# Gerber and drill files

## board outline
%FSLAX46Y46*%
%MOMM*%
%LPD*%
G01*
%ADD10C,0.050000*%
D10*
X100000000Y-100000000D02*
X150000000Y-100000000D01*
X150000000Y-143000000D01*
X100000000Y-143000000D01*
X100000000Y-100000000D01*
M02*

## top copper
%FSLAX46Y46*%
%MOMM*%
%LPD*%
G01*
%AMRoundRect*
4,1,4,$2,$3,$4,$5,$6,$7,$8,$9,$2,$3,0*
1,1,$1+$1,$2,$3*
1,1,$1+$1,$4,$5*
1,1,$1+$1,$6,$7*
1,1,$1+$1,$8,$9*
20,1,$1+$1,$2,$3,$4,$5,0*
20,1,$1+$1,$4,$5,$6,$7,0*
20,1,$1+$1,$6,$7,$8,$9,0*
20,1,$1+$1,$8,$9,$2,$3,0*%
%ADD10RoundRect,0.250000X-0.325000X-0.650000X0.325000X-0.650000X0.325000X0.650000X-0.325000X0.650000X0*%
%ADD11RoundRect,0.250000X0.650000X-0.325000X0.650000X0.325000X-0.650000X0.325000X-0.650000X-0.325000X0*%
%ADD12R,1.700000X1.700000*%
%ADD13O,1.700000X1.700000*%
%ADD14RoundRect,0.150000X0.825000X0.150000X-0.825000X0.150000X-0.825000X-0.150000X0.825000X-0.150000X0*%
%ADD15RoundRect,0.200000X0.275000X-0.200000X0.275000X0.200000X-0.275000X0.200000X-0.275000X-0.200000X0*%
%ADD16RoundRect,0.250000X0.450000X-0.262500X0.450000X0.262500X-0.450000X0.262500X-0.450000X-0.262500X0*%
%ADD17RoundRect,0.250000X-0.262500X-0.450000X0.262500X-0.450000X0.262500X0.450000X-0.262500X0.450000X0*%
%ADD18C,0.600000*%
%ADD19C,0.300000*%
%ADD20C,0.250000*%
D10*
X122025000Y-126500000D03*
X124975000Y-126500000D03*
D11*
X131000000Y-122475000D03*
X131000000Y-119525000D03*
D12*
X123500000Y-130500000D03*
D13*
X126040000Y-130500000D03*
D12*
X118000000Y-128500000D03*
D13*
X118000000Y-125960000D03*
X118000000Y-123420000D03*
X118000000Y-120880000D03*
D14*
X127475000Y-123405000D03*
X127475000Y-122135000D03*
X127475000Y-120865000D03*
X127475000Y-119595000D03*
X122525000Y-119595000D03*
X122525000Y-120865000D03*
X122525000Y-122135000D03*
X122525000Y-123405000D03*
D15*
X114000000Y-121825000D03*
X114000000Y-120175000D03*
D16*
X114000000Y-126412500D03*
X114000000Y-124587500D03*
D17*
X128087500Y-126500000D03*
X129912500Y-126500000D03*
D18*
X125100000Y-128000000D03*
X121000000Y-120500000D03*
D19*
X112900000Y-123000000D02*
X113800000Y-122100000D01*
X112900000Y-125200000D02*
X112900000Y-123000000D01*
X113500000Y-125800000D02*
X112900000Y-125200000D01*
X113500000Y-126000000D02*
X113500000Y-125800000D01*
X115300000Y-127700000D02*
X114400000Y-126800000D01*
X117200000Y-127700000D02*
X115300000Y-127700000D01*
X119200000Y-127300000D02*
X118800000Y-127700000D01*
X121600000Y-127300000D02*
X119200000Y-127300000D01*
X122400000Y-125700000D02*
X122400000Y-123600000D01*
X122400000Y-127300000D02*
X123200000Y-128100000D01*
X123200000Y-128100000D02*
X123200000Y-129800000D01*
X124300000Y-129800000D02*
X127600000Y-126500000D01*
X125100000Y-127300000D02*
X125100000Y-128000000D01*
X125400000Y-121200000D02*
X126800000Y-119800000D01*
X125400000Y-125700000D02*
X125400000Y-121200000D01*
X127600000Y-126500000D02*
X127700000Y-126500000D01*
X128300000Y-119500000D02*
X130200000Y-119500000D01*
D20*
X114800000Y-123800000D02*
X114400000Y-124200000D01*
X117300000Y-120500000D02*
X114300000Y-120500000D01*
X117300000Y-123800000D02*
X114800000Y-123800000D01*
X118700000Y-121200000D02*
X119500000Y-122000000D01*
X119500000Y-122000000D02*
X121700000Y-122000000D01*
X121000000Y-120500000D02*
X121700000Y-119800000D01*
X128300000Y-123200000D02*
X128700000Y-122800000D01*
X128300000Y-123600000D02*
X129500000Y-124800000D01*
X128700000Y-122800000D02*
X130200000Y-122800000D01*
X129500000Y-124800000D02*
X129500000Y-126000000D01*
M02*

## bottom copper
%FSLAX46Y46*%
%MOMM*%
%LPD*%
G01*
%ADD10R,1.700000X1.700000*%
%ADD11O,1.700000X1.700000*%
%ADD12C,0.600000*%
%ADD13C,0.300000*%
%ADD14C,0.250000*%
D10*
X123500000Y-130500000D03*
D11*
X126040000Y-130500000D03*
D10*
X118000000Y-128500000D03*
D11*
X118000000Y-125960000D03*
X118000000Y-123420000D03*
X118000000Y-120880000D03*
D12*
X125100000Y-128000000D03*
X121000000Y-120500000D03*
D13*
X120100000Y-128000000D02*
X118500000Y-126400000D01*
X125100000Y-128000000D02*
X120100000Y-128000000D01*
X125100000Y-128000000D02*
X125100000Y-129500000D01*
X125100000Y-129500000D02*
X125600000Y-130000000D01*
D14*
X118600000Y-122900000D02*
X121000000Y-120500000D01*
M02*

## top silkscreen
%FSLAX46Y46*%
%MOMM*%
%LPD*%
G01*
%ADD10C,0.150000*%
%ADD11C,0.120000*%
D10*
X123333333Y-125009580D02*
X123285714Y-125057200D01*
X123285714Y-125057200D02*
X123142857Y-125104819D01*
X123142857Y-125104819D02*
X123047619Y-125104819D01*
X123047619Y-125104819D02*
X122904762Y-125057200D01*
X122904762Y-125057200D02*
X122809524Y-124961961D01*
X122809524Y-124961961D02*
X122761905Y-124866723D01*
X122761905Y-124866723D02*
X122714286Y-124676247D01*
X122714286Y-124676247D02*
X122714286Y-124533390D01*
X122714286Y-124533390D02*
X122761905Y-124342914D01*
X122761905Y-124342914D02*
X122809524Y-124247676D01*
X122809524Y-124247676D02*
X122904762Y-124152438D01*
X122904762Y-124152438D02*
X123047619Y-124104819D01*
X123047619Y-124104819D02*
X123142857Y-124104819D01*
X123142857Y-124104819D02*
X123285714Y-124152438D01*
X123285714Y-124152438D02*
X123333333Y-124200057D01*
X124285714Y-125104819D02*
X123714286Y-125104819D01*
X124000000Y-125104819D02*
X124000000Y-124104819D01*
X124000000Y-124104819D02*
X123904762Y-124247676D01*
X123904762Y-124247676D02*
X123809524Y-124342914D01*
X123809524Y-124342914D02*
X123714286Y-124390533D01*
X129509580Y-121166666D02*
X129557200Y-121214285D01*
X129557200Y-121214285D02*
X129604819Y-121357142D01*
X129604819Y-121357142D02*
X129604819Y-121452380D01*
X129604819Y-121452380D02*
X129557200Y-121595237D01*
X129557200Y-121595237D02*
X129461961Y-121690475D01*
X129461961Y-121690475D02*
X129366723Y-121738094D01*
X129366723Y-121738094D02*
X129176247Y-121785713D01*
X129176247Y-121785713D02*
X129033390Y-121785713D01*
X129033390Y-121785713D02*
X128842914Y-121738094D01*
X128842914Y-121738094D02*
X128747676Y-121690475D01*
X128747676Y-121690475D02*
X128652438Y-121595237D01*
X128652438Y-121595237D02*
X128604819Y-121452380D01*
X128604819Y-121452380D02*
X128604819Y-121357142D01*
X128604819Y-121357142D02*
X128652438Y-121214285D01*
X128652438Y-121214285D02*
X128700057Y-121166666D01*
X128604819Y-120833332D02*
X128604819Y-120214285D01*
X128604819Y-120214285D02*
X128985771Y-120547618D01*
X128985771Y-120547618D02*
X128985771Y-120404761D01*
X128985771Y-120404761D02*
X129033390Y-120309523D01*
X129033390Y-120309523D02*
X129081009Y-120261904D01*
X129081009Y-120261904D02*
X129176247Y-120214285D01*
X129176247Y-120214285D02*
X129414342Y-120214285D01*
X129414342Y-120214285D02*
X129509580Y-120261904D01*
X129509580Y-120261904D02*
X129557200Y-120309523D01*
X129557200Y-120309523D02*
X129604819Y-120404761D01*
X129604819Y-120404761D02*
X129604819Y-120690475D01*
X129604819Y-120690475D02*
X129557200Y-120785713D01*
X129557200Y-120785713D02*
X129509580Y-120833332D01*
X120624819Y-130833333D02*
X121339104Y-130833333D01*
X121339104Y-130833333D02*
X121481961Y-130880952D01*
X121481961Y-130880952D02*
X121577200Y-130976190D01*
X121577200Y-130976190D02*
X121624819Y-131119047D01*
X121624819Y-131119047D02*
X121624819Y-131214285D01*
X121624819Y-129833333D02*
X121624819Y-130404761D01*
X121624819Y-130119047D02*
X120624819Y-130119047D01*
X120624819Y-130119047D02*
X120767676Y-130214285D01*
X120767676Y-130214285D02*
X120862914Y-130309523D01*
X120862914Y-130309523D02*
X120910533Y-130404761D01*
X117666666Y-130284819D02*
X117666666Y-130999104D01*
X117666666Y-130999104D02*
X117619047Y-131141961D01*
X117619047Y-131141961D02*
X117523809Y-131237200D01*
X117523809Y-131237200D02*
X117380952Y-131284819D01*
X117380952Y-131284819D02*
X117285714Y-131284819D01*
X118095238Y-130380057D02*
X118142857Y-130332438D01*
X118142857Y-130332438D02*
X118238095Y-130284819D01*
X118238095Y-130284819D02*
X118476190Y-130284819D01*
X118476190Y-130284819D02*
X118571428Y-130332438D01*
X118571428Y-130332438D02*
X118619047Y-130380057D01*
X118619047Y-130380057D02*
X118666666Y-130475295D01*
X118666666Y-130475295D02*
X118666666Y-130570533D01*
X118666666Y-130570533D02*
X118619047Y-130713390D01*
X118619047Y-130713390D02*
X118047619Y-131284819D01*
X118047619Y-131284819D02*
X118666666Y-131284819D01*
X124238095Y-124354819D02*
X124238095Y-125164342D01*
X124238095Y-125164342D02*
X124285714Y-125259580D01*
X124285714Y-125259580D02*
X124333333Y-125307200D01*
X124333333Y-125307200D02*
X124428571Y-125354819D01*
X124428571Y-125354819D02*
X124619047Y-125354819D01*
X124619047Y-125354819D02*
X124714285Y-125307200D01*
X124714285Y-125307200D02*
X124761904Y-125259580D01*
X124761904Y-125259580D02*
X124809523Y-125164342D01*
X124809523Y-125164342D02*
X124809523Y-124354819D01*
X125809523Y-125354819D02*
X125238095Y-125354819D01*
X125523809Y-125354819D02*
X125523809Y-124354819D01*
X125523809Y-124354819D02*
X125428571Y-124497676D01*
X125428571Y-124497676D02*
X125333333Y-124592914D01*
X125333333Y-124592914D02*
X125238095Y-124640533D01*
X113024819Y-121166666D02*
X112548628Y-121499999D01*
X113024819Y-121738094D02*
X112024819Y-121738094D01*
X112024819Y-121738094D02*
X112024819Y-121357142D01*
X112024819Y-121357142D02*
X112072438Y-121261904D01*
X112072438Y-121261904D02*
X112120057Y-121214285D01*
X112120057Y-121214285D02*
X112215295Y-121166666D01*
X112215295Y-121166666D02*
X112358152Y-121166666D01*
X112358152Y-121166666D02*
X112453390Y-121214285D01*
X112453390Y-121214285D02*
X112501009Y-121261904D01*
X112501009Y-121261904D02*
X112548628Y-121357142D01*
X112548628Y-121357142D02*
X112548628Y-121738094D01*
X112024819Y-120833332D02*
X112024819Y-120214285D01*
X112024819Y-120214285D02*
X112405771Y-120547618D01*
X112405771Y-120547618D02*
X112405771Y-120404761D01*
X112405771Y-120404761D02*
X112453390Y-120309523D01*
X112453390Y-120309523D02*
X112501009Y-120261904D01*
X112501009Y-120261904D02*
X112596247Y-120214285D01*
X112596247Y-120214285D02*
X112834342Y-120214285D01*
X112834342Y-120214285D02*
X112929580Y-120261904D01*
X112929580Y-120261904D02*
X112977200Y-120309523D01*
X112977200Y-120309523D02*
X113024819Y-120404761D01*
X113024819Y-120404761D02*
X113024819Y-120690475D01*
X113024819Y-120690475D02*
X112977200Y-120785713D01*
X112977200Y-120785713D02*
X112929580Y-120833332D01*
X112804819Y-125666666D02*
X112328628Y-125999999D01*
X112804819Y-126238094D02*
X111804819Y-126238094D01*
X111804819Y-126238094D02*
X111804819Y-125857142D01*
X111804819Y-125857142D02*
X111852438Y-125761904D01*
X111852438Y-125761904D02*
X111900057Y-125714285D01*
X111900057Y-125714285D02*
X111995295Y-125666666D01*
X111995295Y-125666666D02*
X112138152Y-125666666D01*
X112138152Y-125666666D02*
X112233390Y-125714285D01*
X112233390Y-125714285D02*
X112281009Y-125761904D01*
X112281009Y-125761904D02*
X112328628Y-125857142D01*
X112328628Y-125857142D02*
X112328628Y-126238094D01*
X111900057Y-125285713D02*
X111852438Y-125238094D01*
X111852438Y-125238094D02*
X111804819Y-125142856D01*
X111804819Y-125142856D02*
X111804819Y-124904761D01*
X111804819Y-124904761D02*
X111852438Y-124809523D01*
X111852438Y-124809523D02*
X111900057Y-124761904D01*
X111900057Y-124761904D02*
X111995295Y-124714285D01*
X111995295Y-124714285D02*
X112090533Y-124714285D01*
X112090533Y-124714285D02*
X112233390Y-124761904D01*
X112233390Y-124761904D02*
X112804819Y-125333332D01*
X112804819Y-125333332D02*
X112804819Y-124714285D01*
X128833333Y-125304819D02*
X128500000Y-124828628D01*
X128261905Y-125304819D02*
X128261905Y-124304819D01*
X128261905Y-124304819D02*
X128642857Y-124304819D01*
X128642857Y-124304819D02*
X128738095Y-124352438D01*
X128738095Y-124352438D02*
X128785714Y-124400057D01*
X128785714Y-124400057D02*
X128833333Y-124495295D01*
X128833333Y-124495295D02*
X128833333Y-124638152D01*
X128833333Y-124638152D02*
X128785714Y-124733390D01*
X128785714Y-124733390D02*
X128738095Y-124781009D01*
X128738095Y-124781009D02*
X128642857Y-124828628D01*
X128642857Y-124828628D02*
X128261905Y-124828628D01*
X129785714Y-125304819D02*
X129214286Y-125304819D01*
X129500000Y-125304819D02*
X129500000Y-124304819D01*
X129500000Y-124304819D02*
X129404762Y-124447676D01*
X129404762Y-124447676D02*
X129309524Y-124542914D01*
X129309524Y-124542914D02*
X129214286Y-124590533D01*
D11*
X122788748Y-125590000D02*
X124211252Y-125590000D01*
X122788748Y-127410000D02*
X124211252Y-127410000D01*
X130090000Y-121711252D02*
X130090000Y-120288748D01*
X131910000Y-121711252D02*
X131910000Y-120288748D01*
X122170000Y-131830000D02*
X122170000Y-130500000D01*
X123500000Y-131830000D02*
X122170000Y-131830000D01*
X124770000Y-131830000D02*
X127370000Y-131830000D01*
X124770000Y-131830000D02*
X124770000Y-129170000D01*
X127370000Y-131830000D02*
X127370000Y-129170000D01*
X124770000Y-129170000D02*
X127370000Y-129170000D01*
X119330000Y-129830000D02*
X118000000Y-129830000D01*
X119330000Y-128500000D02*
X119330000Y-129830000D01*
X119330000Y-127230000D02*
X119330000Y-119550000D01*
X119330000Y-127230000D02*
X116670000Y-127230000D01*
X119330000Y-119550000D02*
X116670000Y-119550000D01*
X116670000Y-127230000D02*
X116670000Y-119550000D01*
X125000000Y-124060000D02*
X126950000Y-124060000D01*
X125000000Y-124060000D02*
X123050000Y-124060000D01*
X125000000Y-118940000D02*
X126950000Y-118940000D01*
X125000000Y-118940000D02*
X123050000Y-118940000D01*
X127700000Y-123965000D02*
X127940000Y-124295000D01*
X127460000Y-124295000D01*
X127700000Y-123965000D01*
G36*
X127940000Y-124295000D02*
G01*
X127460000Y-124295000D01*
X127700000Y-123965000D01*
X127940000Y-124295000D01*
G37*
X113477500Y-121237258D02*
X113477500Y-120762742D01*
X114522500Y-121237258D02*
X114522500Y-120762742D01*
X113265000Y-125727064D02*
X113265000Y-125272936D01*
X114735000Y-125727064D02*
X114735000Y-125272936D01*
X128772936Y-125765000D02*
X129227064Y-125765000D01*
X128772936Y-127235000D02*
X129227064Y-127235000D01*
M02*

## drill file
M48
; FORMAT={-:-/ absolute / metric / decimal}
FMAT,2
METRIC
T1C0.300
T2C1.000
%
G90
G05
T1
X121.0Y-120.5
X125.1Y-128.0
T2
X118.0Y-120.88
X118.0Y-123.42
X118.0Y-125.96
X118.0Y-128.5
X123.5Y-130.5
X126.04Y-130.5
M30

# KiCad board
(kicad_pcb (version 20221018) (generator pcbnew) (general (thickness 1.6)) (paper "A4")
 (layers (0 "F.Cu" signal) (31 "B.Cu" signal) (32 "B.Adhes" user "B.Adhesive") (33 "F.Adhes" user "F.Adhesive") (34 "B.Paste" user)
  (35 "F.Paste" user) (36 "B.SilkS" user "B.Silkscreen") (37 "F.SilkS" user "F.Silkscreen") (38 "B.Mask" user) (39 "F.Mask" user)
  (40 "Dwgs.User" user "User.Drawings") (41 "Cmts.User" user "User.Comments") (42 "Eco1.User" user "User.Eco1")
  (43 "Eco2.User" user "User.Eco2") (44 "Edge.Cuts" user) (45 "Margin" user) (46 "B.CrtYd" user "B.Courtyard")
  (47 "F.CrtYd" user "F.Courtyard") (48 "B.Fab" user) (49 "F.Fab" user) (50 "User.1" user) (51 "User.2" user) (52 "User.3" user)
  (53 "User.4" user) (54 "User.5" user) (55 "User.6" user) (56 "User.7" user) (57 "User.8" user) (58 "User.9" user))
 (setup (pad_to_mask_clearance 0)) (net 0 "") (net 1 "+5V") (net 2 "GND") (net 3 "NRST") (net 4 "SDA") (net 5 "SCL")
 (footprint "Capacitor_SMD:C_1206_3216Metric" (layer "F.Cu") (at 123.5 126.5)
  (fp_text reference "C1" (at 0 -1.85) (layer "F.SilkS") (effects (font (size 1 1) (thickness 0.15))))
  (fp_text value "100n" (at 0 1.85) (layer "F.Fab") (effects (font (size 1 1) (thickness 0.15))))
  (fp_line (start -0.711252 -0.91) (end 0.711252 -0.91) (stroke (width 0.12) (type solid)) (layer "F.SilkS"))
  (fp_line (start -0.711252 0.91) (end 0.711252 0.91) (stroke (width 0.12) (type solid)) (layer "F.SilkS"))
  (pad "1" smd roundrect (at -1.475 0) (size 1.15 1.8) (layers "F.Cu" "F.Paste" "F.Mask") (roundrect_rratio 0.217391) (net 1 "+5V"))
  (pad "2" smd roundrect (at 1.475 0) (size 1.15 1.8) (layers "F.Cu" "F.Paste" "F.Mask") (roundrect_rratio 0.217391) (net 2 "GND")))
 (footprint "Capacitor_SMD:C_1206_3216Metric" (layer "F.Cu") (at 131 121 90)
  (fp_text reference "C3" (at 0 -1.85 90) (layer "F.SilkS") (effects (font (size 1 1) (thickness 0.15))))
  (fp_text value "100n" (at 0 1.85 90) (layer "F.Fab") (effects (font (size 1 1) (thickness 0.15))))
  (fp_line (start -0.711252 -0.91) (end 0.711252 -0.91) (stroke (width 0.12) (type solid)) (layer "F.SilkS"))
  (fp_line (start -0.711252 0.91) (end 0.711252 0.91) (stroke (width 0.12) (type solid)) (layer "F.SilkS"))
  (pad "1" smd roundrect (at -1.475 0 90) (size 1.15 1.8) (layers "F.Cu" "F.Paste" "F.Mask") (roundrect_rratio 0.217391) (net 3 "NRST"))
  (pad "2" smd roundrect (at 1.475 0 90) (size 1.15 1.8) (layers "F.Cu" "F.Paste" "F.Mask") (roundrect_rratio 0.217391) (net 2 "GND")))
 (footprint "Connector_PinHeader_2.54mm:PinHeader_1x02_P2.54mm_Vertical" (layer "F.Cu") (at 123.5 130.5 90)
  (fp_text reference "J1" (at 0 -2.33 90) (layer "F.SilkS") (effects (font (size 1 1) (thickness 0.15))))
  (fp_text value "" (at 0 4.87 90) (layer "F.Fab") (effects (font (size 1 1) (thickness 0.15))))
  (fp_line (start -1.33 -1.33) (end 0 -1.33) (stroke (width 0.12) (type solid)) (layer "F.SilkS"))
  (fp_line (start -1.33 0) (end -1.33 -1.33) (stroke (width 0.12) (type solid)) (layer "F.SilkS"))
  (fp_line (start -1.33 1.27) (end -1.33 3.87) (stroke (width 0.12) (type solid)) (layer "F.SilkS"))
  (fp_line (start -1.33 1.27) (end 1.33 1.27) (stroke (width 0.12) (type solid)) (layer "F.SilkS"))
  (fp_line (start -1.33 3.87) (end 1.33 3.87) (stroke (width 0.12) (type solid)) (layer "F.SilkS"))
  (fp_line (start 1.33 1.27) (end 1.33 3.87) (stroke (width 0.12) (type solid)) (layer "F.SilkS"))
  (pad "1" thru_hole rect (at 0 0 90) (size 1.7 1.7) (drill 1) (layers "*.Cu" "*.Mask") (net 1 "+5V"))
  (pad "2" thru_hole oval (at 0 2.54 90) (size 1.7 1.7) (drill 1) (layers "*.Cu" "*.Mask") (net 2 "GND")))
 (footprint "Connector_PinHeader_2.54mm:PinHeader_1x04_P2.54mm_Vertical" (layer "F.Cu") (at 118 128.5 180)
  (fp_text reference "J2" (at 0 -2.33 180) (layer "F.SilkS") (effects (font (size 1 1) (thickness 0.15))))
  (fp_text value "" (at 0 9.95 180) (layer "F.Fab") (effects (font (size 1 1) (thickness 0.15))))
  (fp_line (start -1.33 -1.33) (end 0 -1.33) (stroke (width 0.12) (type solid)) (layer "F.SilkS"))
  (fp_line (start -1.33 0) (end -1.33 -1.33) (stroke (width 0.12) (type solid)) (layer "F.SilkS"))
  (fp_line (start -1.33 1.27) (end -1.33 8.95) (stroke (width 0.12) (type solid)) (layer "F.SilkS"))
  (fp_line (start -1.33 1.27) (end 1.33 1.27) (stroke (width 0.12) (type solid)) (layer "F.SilkS"))
  (fp_line (start -1.33 8.95) (end 1.33 8.95) (stroke (width 0.12) (type solid)) (layer "F.SilkS"))
  (fp_line (start 1.33 1.27) (end 1.33 8.95) (stroke (width 0.12) (type solid)) (layer "F.SilkS"))
  (pad "1" thru_hole rect (at 0 0 180) (size 1.7 1.7) (drill 1) (layers "*.Cu" "*.Mask") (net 1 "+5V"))
  (pad "2" thru_hole oval (at 0 2.54 180) (size 1.7 1.7) (drill 1) (layers "*.Cu" "*.Mask") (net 2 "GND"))
  (pad "3" thru_hole oval (at 0 5.08 180) (size 1.7 1.7) (drill 1) (layers "*.Cu" "*.Mask") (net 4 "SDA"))
  (pad "4" thru_hole oval (at 0 7.62 180) (size 1.7 1.7) (drill 1) (layers "*.Cu" "*.Mask") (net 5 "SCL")))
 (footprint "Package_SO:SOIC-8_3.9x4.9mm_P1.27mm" (layer "F.Cu") (at 125 121.5 180)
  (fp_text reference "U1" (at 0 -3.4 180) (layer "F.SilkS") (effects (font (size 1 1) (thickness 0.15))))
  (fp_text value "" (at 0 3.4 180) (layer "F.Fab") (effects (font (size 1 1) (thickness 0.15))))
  (fp_line (start 0 -2.56) (end -1.95 -2.56) (stroke (width 0.12) (type solid)) (layer "F.SilkS"))
  (fp_line (start 0 -2.56) (end 1.95 -2.56) (stroke (width 0.12) (type solid)) (layer "F.SilkS"))
  (fp_line (start 0 2.56) (end -1.95 2.56) (stroke (width 0.12) (type solid)) (layer "F.SilkS"))
  (fp_line (start 0 2.56) (end 1.95 2.56) (stroke (width 0.12) (type solid)) (layer "F.SilkS"))
  (fp_poly
   (pts (xy -2.7 -2.465) (xy -2.94 -2.795) (xy -2.46 -2.795) (xy -2.7 -2.465)) (stroke (width 0.12) (type solid)) (fill solid)
   (layer "F.SilkS"))
  (pad "1" smd roundrect (at -2.475 -1.905 180) (size 1.95 0.6) (layers "F.Cu" "F.Paste" "F.Mask") (roundrect_rratio 0.25) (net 3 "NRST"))
  (pad "2" smd roundrect (at -2.475 -0.635 180) (size 1.95 0.6) (layers "F.Cu" "F.Paste" "F.Mask") (roundrect_rratio 0.25))
  (pad "3" smd roundrect (at -2.475 0.635 180) (size 1.95 0.6) (layers "F.Cu" "F.Paste" "F.Mask") (roundrect_rratio 0.25))
  (pad "4" smd roundrect (at -2.475 1.905 180) (size 1.95 0.6) (layers "F.Cu" "F.Paste" "F.Mask") (roundrect_rratio 0.25) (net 2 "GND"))
  (pad "5" smd roundrect (at 2.475 1.905 180) (size 1.95 0.6) (layers "F.Cu" "F.Paste" "F.Mask") (roundrect_rratio 0.25) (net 4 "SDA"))
  (pad "6" smd roundrect (at 2.475 0.635 180) (size 1.95 0.6) (layers "F.Cu" "F.Paste" "F.Mask") (roundrect_rratio 0.25))
  (pad "7" smd roundrect (at 2.475 -0.635 180) (size 1.95 0.6) (layers "F.Cu" "F.Paste" "F.Mask") (roundrect_rratio 0.25) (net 5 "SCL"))
  (pad "8" smd roundrect (at 2.475 -1.905 180) (size 1.95 0.6) (layers "F.Cu" "F.Paste" "F.Mask") (roundrect_rratio 0.25) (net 1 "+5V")))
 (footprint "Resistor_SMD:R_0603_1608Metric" (layer "F.Cu") (at 114 121 90)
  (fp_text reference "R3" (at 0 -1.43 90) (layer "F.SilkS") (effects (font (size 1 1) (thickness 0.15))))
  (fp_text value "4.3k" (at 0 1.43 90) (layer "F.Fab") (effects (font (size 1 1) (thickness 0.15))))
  (fp_line (start -0.237258 -0.5225) (end 0.237258 -0.5225) (stroke (width 0.12) (type solid)) (layer "F.SilkS"))
  (fp_line (start -0.237258 0.5225) (end 0.237258 0.5225) (stroke (width 0.12) (type solid)) (layer "F.SilkS"))
  (pad "1" smd roundrect (at -0.825 0 90) (size 0.8 0.95) (layers "F.Cu" "F.Paste" "F.Mask") (roundrect_rratio 0.25) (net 1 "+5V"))
  (pad "2" smd roundrect (at 0.825 0 90) (size 0.8 0.95) (layers "F.Cu" "F.Paste" "F.Mask") (roundrect_rratio 0.25) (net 5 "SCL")))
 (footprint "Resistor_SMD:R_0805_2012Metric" (layer "F.Cu") (at 114 125.5 90)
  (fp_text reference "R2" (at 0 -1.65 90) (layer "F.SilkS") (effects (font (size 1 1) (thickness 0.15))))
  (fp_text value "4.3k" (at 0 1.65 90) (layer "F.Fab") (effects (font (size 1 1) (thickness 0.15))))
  (fp_line (start -0.227064 -0.735) (end 0.227064 -0.735) (stroke (width 0.12) (type solid)) (layer "F.SilkS"))
  (fp_line (start -0.227064 0.735) (end 0.227064 0.735) (stroke (width 0.12) (type solid)) (layer "F.SilkS"))
  (pad "1" smd roundrect (at -0.9125 0 90) (size 1.025 1.4) (layers "F.Cu" "F.Paste" "F.Mask") (roundrect_rratio 0.243902) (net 1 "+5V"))
  (pad "2" smd roundrect (at 0.9125 0 90) (size 1.025 1.4) (layers "F.Cu" "F.Paste" "F.Mask") (roundrect_rratio 0.243902) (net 4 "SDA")))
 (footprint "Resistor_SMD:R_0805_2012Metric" (layer "F.Cu") (at 129 126.5)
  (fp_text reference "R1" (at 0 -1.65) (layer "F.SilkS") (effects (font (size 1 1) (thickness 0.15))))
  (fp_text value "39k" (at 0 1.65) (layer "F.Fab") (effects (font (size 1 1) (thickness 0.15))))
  (fp_line (start -0.227064 -0.735) (end 0.227064 -0.735) (stroke (width 0.12) (type solid)) (layer "F.SilkS"))
  (fp_line (start -0.227064 0.735) (end 0.227064 0.735) (stroke (width 0.12) (type solid)) (layer "F.SilkS"))
  (pad "1" smd roundrect (at -0.9125 0) (size 1.025 1.4) (layers "F.Cu" "F.Paste" "F.Mask") (roundrect_rratio 0.243902) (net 1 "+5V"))
  (pad "2" smd roundrect (at 0.9125 0) (size 1.025 1.4) (layers "F.Cu" "F.Paste" "F.Mask") (roundrect_rratio 0.243902) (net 3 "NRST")))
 (gr_rect (start 100 100) (end 150 143) (stroke (width 0.05) (type default)) (fill none) (layer "Edge.Cuts"))
 (segment (start 112.9 123) (end 113.8 122.1) (width 0.3) (layer "F.Cu") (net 1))
 (segment (start 112.9 125.2) (end 112.9 123) (width 0.3) (layer "F.Cu") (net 1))
 (segment (start 113.5 125.8) (end 112.9 125.2) (width 0.3) (layer "F.Cu") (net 1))
 (segment (start 113.5 126) (end 113.5 125.8) (width 0.3) (layer "F.Cu") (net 1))
 (segment (start 115.3 127.7) (end 114.4 126.8) (width 0.3) (layer "F.Cu") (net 1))
 (segment (start 117.2 127.7) (end 115.3 127.7) (width 0.3) (layer "F.Cu") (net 1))
 (segment (start 119.2 127.3) (end 118.8 127.7) (width 0.3) (layer "F.Cu") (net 1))
 (segment (start 121.6 127.3) (end 119.2 127.3) (width 0.3) (layer "F.Cu") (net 1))
 (segment (start 122.4 125.7) (end 122.4 123.6) (width 0.3) (layer "F.Cu") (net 1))
 (segment (start 122.4 127.3) (end 123.2 128.1) (width 0.3) (layer "F.Cu") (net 1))
 (segment (start 123.2 128.1) (end 123.2 129.8) (width 0.3) (layer "F.Cu") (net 1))
 (segment (start 124.3 129.8) (end 127.6 126.5) (width 0.3) (layer "F.Cu") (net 1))
 (segment (start 125.1 127.3) (end 125.1 128) (width 0.3) (layer "F.Cu") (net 2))
 (segment (start 125.4 121.2) (end 126.8 119.8) (width 0.3) (layer "F.Cu") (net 2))
 (segment (start 125.4 125.7) (end 125.4 121.2) (width 0.3) (layer "F.Cu") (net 2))
 (segment (start 127.6 126.5) (end 127.7 126.5) (width 0.3) (layer "F.Cu") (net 1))
 (segment (start 128.3 119.5) (end 130.2 119.5) (width 0.3) (layer "F.Cu") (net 2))
 (via (at 125.1 128) (size 0.6) (drill 0.3) (layers "F.Cu" "B.Cu") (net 2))
 (segment (start 114.8 123.8) (end 114.4 124.2) (width 0.25) (layer "F.Cu") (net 4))
 (segment (start 117.3 120.5) (end 114.3 120.5) (width 0.25) (layer "F.Cu") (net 5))
 (segment (start 117.3 123.8) (end 114.8 123.8) (width 0.25) (layer "F.Cu") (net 4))
 (segment (start 118.7 121.2) (end 119.5 122) (width 0.25) (layer "F.Cu") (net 5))
 (segment (start 119.5 122) (end 121.7 122) (width 0.25) (layer "F.Cu") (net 5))
 (segment (start 120.1 128) (end 118.5 126.4) (width 0.3) (layer "B.Cu") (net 2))
 (segment (start 121 120.5) (end 121.7 119.8) (width 0.25) (layer "F.Cu") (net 4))
 (segment (start 125.1 128) (end 120.1 128) (width 0.3) (layer "B.Cu") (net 2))
 (segment (start 125.1 128) (end 125.1 129.5) (width 0.3) (layer "B.Cu") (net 2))
 (segment (start 125.1 129.5) (end 125.6 130) (width 0.3) (layer "B.Cu") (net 2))
 (segment (start 128.3 123.2) (end 128.7 122.8) (width 0.25) (layer "F.Cu") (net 3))
 (segment (start 128.3 123.6) (end 129.5 124.8) (width 0.25) (layer "F.Cu") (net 3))
 (segment (start 128.7 122.8) (end 130.2 122.8) (width 0.25) (layer "F.Cu") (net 3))
 (segment (start 129.5 124.8) (end 129.5 126) (width 0.25) (layer "F.Cu") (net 3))
 (via (at 121 120.5) (size 0.6) (drill 0.3) (layers "F.Cu" "B.Cu") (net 4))
 (segment (start 118.6 122.9) (end 121 120.5) (width 0.25) (layer "B.Cu") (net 4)))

